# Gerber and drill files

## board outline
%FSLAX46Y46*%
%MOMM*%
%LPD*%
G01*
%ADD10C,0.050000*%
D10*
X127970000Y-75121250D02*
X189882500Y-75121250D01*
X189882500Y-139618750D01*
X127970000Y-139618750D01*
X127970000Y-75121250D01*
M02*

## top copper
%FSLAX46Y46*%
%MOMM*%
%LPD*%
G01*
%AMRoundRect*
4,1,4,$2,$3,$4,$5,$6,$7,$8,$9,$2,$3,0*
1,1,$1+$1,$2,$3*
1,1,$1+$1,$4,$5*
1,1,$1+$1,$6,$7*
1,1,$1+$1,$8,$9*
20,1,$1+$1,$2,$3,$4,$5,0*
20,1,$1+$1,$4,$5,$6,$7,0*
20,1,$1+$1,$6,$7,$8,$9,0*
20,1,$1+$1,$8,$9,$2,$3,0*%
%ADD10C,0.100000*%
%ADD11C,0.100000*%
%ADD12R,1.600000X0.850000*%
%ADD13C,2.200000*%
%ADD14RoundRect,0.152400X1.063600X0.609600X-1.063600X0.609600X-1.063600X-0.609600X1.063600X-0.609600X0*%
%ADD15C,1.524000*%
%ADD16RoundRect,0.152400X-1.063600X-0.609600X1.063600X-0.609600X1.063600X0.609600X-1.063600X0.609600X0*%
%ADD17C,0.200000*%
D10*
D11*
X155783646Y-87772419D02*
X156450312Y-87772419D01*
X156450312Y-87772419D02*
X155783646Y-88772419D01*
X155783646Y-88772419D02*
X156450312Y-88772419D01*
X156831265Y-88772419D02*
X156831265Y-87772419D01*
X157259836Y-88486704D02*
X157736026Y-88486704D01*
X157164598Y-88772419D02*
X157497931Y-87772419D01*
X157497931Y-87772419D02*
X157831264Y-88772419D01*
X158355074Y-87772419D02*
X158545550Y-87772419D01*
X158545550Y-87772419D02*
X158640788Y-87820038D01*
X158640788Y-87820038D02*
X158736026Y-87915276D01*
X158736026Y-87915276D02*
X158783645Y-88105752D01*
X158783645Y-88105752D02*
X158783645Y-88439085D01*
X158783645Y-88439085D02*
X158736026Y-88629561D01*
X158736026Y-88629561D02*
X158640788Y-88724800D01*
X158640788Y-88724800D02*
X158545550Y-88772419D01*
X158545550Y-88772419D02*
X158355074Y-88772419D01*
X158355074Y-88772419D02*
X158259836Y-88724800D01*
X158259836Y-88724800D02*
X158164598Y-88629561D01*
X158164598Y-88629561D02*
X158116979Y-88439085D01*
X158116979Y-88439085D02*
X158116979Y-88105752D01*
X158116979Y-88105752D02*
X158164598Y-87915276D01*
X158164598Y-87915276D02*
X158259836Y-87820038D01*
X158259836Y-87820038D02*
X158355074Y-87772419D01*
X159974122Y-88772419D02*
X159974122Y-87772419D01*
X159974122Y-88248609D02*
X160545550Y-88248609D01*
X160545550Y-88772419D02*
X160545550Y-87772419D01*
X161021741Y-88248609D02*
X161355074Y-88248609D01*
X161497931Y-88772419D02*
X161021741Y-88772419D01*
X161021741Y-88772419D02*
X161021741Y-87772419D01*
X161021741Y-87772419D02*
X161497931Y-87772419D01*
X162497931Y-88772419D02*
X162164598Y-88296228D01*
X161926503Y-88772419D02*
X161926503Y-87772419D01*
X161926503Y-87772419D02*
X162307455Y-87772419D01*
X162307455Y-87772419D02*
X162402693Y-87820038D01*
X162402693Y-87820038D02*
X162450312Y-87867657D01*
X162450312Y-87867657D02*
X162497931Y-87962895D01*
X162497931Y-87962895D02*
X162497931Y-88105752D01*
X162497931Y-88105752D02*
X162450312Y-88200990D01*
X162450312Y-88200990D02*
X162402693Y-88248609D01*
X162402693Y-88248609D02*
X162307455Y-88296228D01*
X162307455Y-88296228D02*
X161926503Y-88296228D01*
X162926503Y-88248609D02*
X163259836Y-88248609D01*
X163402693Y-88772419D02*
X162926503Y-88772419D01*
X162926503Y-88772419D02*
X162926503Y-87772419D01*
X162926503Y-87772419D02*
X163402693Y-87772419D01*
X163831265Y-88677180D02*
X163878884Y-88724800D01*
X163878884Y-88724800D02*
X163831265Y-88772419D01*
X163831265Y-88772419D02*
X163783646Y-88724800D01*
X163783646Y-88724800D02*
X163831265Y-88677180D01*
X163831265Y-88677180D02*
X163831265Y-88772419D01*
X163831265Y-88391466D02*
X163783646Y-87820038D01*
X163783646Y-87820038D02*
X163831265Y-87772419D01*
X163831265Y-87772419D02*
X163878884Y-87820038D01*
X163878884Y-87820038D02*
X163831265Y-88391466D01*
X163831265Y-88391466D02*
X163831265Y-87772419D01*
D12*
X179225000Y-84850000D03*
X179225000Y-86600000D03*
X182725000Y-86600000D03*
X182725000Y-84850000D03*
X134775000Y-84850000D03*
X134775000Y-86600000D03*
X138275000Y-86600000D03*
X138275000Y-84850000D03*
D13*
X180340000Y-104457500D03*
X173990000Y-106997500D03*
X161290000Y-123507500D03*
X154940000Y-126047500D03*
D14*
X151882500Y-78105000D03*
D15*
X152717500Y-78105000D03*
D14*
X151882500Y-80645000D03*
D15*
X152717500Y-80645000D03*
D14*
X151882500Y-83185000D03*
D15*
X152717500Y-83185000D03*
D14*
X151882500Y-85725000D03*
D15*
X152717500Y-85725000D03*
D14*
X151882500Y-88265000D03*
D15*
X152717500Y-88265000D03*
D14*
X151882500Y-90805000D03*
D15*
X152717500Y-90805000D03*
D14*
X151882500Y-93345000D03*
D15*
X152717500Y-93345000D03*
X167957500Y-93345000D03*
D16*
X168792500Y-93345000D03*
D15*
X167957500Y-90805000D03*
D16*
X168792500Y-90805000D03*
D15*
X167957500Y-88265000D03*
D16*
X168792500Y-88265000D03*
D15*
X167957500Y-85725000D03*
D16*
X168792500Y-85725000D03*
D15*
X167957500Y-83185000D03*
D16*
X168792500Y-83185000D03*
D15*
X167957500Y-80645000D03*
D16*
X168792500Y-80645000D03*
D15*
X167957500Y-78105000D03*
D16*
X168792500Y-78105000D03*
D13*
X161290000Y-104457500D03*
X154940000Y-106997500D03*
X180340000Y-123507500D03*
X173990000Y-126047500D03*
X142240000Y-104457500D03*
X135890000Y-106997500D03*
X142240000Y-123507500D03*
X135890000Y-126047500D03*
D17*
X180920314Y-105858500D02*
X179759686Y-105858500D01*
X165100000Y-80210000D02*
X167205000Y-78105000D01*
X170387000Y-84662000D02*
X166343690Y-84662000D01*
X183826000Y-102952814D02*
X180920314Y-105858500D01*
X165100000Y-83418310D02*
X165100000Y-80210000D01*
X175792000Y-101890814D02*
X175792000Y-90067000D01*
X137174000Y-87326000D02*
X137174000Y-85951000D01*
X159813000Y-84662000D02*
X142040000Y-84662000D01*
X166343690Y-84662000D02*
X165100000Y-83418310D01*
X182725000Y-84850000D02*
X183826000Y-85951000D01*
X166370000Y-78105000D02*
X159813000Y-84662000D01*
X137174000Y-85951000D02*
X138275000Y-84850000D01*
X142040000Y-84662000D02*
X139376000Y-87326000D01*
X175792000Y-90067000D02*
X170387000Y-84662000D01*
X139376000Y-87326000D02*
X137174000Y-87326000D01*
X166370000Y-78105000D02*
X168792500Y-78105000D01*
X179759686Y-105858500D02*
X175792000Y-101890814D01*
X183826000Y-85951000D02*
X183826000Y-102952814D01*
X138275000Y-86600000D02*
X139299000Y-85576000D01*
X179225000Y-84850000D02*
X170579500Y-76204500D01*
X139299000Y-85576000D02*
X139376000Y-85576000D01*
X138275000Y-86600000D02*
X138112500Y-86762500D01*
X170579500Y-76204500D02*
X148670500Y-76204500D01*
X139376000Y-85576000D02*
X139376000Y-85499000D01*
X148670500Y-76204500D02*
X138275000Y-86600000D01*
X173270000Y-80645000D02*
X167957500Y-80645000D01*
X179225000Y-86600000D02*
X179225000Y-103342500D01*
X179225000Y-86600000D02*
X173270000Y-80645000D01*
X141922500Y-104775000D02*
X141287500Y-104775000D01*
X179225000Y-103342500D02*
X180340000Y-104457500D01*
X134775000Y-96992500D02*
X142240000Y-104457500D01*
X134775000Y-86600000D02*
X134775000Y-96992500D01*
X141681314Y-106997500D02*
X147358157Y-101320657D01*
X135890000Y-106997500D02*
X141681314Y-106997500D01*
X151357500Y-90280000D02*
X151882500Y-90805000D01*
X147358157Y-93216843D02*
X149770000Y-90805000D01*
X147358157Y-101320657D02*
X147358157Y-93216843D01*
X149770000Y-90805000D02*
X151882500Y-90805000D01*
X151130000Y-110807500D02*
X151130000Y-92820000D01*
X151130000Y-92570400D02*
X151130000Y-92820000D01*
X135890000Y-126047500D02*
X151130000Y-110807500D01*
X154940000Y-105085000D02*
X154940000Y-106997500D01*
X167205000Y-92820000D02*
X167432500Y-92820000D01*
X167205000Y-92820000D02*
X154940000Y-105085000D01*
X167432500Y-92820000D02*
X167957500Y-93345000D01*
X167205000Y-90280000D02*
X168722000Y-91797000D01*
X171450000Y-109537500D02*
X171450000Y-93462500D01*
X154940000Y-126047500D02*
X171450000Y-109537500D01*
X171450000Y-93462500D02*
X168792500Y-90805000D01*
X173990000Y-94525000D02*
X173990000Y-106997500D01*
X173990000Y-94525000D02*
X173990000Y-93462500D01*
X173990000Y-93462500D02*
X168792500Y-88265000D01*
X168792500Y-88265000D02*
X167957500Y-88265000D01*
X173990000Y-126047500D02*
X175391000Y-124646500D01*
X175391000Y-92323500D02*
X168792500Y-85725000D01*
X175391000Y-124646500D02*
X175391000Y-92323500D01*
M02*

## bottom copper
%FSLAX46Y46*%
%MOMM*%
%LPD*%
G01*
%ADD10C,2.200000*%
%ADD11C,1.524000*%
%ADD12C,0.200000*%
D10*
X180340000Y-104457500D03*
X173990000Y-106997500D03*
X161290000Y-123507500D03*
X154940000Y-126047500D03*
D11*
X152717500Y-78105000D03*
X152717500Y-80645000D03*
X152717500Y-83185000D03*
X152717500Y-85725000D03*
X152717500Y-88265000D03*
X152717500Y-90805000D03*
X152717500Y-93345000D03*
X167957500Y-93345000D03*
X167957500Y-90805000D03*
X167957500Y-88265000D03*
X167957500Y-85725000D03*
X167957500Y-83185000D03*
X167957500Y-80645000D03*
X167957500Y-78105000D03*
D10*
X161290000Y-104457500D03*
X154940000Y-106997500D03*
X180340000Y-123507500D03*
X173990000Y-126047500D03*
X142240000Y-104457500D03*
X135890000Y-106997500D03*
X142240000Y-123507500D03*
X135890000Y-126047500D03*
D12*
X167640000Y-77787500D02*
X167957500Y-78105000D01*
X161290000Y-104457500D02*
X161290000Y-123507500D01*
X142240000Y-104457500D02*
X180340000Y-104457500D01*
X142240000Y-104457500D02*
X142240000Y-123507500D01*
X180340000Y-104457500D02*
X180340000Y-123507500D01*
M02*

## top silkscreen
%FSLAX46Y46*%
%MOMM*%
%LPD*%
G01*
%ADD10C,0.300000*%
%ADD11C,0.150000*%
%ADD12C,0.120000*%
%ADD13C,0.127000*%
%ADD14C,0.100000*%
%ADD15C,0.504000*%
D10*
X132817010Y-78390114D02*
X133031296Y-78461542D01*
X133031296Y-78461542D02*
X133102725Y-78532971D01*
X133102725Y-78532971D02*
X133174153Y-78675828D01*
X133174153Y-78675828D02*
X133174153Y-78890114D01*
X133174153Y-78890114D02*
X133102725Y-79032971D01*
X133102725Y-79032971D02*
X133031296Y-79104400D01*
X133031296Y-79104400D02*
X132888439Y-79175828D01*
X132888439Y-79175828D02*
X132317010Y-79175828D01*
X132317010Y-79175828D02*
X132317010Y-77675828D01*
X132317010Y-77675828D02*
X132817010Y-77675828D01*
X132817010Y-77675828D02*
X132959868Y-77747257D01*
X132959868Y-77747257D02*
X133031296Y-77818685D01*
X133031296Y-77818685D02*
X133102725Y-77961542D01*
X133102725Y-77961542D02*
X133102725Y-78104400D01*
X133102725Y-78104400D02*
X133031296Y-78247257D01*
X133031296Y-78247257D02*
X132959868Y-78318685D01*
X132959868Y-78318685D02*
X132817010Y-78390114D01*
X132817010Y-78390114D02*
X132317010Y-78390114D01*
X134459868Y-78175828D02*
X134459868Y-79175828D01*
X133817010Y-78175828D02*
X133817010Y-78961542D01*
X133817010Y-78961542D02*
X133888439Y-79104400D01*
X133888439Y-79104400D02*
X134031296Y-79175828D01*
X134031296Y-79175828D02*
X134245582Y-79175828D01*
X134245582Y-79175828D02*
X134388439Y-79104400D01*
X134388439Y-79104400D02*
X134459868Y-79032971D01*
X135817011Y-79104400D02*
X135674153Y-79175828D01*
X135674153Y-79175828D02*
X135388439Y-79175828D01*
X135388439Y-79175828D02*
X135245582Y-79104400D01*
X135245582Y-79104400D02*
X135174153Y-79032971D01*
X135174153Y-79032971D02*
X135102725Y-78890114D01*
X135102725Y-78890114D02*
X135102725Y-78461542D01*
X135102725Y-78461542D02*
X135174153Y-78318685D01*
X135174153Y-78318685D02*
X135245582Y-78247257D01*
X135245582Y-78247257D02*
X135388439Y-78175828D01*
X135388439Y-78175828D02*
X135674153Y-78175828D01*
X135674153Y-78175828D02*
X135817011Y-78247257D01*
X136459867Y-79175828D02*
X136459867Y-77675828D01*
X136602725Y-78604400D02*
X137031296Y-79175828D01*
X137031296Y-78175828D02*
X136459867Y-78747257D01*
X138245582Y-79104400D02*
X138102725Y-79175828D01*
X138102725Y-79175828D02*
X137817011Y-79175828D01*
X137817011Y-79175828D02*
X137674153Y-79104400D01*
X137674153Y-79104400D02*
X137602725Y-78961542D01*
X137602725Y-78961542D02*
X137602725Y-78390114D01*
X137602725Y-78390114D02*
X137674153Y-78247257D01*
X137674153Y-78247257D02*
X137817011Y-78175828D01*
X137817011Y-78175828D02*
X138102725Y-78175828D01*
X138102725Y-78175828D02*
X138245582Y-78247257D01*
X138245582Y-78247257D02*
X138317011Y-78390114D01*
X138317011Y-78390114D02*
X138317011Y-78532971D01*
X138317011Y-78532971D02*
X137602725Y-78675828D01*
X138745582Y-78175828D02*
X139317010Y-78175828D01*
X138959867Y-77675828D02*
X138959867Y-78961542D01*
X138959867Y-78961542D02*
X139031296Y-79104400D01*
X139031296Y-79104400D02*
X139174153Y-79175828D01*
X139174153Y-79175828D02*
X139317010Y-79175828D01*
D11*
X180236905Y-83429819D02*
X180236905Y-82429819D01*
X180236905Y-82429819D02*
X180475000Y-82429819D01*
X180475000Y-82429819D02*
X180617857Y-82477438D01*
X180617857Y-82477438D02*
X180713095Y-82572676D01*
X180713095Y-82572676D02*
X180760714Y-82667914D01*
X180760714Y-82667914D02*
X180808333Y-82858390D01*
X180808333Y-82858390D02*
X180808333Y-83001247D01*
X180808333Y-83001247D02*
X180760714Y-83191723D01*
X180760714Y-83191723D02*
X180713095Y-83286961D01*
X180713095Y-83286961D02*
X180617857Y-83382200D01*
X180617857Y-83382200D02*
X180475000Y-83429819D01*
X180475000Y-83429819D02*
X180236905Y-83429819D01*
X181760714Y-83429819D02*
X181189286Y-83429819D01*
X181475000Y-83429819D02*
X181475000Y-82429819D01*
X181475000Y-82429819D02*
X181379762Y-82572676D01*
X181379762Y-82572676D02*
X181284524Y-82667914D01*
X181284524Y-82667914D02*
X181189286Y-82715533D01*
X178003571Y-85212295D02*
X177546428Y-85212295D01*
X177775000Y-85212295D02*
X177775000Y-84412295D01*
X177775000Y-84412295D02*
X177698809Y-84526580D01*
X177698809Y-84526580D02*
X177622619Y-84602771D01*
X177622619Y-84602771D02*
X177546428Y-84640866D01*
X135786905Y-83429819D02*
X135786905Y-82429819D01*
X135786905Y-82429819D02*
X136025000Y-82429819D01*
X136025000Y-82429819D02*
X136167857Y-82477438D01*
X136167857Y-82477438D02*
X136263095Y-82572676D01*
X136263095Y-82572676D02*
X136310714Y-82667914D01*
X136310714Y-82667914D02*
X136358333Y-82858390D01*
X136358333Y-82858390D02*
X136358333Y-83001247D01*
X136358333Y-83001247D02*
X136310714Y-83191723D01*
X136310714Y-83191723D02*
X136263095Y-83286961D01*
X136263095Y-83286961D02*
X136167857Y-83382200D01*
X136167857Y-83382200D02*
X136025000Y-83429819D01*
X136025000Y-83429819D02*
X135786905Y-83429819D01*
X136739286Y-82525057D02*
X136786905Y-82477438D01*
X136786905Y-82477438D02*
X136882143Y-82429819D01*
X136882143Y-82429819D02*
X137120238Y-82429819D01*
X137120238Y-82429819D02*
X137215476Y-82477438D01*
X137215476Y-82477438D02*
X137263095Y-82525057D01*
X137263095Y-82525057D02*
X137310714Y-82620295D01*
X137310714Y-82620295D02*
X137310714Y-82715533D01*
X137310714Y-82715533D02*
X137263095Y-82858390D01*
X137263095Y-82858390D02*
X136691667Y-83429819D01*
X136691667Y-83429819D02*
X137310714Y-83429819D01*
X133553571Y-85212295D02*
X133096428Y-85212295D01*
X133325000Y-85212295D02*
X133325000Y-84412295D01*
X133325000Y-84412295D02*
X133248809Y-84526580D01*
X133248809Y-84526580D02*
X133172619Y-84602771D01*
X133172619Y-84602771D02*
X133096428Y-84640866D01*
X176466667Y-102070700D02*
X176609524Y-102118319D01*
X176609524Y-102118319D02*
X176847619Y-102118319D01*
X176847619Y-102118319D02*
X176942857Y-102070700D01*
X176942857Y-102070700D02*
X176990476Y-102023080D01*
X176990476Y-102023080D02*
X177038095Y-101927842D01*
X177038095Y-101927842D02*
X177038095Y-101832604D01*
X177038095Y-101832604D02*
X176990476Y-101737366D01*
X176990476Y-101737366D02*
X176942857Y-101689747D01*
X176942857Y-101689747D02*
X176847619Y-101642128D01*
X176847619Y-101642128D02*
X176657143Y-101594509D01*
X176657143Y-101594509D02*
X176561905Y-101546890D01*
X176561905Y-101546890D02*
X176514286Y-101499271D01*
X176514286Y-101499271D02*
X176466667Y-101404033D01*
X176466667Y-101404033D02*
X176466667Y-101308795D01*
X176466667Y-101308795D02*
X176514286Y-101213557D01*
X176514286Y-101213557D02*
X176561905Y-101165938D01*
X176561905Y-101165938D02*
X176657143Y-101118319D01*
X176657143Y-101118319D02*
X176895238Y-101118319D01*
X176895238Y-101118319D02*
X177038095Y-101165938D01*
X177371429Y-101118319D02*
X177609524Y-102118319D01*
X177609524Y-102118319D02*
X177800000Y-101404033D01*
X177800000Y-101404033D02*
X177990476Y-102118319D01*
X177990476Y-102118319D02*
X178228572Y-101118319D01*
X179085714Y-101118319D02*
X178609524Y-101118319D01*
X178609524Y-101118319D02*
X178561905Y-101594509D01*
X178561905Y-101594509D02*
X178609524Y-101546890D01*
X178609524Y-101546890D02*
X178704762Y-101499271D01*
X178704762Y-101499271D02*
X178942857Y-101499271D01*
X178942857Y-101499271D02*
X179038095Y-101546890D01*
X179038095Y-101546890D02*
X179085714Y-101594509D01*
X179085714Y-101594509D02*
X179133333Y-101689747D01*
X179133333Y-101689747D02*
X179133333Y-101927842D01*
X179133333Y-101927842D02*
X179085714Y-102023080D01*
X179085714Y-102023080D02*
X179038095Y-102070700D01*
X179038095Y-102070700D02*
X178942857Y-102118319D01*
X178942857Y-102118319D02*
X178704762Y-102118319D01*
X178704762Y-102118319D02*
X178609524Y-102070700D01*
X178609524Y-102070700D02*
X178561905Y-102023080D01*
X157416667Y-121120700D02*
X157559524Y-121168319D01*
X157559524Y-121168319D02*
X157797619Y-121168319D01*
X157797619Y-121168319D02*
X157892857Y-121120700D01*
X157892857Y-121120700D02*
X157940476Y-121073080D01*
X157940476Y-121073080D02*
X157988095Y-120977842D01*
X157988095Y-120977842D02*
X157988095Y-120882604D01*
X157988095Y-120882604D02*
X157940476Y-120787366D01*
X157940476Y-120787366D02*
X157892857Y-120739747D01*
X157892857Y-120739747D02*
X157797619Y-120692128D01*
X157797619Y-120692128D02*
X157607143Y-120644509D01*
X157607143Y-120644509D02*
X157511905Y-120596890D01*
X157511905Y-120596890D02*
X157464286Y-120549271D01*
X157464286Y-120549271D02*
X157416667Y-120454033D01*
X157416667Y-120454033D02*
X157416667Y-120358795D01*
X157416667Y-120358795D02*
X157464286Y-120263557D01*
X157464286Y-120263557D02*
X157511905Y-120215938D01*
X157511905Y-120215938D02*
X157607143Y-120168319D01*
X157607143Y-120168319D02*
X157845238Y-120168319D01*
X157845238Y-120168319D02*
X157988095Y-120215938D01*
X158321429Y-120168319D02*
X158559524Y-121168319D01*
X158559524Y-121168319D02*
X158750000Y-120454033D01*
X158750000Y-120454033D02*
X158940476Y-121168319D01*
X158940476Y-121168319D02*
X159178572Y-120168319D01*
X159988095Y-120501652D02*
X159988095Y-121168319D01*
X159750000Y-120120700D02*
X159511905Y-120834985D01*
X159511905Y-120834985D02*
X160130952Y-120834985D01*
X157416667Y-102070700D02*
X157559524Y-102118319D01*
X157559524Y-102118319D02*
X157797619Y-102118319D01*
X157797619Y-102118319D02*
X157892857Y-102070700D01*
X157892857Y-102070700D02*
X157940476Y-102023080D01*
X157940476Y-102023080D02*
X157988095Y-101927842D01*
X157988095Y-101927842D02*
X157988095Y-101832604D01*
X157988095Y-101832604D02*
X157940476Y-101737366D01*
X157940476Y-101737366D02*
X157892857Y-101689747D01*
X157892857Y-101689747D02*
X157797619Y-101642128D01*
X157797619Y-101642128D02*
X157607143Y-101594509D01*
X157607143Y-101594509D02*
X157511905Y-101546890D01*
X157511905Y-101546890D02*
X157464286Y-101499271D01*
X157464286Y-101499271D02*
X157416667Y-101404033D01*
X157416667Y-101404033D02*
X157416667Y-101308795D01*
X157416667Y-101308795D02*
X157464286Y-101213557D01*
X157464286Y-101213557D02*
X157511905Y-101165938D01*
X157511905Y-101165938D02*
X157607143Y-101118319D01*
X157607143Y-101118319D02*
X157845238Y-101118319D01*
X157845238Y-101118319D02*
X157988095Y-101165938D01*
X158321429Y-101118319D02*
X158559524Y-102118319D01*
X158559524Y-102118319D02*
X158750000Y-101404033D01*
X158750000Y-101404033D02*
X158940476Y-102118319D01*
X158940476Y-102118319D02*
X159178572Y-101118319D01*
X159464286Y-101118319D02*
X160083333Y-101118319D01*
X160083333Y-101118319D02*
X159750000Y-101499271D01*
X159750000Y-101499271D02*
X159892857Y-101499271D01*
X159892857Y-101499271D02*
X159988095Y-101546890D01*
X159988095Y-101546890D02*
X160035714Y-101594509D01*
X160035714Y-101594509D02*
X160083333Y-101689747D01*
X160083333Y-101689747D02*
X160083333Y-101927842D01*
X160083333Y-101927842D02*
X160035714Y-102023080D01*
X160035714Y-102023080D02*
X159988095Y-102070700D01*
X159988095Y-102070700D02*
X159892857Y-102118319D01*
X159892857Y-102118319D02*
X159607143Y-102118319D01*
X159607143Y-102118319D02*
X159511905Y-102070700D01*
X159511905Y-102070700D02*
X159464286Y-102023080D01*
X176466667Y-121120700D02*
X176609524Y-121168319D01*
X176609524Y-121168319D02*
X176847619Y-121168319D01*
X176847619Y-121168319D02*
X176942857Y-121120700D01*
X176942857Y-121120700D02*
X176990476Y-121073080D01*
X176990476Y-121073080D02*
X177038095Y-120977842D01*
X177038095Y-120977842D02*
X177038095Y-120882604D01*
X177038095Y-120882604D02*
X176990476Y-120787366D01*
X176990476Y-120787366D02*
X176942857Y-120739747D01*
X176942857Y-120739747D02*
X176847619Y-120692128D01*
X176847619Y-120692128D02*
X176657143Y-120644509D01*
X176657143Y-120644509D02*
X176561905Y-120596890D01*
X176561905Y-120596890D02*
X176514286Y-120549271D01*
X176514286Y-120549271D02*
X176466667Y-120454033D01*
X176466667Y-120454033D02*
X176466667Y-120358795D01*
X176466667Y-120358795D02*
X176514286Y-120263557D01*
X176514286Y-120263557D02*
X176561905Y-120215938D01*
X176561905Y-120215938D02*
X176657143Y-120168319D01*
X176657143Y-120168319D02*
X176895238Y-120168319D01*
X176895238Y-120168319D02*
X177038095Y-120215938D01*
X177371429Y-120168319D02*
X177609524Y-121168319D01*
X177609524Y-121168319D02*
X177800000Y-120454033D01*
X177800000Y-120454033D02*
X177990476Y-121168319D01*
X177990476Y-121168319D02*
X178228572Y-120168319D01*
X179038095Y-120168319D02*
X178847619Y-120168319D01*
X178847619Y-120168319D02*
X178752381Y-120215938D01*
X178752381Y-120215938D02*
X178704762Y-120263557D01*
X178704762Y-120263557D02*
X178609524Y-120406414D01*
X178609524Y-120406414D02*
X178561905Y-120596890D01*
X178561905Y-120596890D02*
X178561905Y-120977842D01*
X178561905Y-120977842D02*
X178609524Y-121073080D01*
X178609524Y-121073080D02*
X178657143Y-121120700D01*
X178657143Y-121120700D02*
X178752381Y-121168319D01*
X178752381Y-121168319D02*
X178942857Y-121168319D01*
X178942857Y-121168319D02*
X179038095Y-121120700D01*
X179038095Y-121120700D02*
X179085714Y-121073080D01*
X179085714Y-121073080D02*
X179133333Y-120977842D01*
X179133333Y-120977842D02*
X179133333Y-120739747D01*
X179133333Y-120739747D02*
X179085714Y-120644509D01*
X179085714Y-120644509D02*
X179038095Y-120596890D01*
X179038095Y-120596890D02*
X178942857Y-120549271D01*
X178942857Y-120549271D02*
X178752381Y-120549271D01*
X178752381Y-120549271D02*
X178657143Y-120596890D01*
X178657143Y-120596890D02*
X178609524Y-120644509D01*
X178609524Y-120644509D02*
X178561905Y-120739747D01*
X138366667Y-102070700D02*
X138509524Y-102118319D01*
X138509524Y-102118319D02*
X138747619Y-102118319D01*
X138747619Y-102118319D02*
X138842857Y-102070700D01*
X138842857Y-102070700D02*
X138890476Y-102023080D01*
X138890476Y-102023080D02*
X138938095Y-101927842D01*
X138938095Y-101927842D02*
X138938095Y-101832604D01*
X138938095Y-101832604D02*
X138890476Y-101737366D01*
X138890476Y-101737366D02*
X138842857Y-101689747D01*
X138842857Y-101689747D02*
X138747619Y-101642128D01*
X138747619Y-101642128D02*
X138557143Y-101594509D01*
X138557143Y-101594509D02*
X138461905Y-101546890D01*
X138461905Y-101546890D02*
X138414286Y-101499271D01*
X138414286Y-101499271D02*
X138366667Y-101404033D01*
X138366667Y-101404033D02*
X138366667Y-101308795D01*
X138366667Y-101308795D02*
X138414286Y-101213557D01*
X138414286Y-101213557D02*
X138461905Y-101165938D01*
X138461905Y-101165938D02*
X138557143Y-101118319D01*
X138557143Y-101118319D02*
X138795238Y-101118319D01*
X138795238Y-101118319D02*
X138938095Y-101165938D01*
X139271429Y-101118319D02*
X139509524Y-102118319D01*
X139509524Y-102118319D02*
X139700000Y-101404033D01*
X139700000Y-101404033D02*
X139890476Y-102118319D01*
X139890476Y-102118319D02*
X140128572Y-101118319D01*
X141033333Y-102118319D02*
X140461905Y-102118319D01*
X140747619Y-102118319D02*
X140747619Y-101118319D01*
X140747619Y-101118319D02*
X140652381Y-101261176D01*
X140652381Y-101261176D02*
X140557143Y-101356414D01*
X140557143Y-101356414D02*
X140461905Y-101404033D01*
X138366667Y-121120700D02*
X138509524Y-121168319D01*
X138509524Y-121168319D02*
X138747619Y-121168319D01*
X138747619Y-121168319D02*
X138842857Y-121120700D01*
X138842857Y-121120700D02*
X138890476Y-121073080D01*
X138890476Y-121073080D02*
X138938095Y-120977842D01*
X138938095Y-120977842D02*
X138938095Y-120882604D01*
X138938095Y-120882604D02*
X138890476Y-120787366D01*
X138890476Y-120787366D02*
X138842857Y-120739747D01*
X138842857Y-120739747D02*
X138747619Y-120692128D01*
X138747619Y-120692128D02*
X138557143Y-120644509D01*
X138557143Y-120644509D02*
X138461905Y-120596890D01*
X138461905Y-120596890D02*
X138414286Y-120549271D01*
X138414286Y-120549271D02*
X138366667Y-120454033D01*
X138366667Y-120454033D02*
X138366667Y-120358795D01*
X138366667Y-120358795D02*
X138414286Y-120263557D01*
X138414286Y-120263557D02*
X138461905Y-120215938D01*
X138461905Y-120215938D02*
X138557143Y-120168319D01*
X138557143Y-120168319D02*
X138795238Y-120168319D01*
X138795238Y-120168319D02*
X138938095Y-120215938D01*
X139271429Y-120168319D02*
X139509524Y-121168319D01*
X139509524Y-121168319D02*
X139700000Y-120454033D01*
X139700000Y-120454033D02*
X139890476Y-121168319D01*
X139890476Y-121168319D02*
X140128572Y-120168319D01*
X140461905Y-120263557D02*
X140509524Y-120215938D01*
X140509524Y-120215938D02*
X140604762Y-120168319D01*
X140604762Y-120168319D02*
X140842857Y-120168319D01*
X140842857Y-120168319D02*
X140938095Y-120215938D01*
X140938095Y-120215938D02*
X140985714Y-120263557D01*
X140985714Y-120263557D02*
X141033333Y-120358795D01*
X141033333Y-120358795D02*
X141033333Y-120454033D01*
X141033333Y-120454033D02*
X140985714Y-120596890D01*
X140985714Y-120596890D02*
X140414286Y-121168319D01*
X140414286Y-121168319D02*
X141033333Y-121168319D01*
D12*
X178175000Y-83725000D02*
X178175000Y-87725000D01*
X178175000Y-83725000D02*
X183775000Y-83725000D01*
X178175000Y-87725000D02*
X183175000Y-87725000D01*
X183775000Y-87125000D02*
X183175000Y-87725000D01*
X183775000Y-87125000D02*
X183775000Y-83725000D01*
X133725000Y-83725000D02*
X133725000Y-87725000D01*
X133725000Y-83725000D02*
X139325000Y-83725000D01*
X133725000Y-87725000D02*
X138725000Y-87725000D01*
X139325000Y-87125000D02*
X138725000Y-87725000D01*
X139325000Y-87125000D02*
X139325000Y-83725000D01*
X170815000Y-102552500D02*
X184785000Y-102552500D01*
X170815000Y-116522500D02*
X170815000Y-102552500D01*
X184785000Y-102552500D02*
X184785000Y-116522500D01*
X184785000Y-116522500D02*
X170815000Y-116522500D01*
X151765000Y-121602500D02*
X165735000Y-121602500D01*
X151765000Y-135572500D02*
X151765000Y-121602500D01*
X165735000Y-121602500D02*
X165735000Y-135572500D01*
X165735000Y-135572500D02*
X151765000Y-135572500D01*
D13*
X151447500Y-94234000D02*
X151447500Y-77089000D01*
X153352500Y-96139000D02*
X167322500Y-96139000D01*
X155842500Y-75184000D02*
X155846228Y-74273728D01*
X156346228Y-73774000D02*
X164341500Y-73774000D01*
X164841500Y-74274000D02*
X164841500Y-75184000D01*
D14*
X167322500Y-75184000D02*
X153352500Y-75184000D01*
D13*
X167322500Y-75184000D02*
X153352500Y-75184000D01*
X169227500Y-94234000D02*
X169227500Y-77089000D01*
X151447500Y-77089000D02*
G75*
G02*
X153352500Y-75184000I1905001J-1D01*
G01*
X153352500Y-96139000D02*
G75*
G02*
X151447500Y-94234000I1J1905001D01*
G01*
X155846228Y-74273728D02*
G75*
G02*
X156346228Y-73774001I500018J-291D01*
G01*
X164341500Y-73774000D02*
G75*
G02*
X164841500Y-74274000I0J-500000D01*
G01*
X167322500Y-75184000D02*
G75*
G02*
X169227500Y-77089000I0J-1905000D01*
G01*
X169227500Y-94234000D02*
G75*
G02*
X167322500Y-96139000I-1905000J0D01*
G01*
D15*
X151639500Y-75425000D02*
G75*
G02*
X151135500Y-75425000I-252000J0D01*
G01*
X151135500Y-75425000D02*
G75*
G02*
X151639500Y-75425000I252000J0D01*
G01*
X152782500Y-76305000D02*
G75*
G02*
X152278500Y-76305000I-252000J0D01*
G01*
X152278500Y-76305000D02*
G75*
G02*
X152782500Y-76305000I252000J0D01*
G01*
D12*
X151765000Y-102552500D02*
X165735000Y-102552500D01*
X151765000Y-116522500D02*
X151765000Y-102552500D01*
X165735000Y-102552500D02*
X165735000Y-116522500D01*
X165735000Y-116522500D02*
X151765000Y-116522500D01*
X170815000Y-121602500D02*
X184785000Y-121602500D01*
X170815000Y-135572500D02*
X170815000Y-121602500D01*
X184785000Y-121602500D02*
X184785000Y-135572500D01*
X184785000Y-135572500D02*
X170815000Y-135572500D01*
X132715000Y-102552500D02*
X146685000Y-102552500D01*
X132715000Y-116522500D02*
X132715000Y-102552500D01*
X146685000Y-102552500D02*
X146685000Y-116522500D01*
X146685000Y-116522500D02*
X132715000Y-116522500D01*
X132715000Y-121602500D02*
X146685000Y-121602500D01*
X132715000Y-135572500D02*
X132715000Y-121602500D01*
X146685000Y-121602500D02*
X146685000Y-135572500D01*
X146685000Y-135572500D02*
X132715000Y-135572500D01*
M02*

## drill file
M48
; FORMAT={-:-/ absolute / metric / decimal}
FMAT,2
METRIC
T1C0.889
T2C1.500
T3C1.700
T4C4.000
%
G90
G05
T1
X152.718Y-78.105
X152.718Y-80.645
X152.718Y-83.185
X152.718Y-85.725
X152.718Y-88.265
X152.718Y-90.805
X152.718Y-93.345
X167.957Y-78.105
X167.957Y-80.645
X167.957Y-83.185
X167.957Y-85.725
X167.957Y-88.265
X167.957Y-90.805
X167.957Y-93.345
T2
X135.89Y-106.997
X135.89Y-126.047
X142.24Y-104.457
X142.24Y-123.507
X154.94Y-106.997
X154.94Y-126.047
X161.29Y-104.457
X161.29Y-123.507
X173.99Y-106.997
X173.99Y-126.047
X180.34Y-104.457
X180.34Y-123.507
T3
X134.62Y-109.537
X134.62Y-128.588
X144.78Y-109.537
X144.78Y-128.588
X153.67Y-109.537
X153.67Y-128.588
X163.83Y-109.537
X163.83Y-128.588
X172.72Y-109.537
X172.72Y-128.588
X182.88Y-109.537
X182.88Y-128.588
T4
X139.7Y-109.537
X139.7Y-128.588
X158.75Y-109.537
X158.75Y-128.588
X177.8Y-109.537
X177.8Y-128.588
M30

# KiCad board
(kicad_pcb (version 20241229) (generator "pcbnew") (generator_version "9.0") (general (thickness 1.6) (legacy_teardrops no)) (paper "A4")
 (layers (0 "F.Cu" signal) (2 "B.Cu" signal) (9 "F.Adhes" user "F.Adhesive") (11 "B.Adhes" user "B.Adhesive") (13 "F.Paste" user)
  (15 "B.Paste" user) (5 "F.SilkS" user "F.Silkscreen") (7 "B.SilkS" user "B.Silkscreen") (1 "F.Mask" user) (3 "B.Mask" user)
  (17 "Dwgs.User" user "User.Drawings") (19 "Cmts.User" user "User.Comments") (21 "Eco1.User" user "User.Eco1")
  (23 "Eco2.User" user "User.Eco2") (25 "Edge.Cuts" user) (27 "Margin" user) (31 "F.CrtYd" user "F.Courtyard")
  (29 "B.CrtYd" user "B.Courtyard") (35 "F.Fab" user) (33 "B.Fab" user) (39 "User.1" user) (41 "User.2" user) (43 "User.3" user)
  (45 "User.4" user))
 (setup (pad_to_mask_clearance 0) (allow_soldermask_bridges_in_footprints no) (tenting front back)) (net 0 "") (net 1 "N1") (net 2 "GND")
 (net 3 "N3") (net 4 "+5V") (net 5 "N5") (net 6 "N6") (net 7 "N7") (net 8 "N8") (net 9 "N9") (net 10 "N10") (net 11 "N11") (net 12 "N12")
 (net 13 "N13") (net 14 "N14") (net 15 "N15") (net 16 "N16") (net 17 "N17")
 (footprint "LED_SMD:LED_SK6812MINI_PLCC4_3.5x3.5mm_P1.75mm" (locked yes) (layer "F.Cu") (at 180.975 85.725)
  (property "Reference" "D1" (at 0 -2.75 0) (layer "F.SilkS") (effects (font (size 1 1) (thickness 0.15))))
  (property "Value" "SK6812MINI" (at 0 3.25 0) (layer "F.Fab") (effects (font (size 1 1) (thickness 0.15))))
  (fp_line (start -2.8 -2) (end -2.8 2) (stroke (width 0.12) (type default)) (layer "F.SilkS"))
  (fp_line (start -2.8 -2) (end 2.8 -2) (stroke (width 0.12) (type solid)) (layer "F.SilkS"))
  (fp_line (start -2.8 2) (end 2.2 2) (stroke (width 0.12) (type solid)) (layer "F.SilkS"))
  (fp_line (start 2.8 1.4) (end 2.2 2) (stroke (width 0.12) (type default)) (layer "F.SilkS"))
  (fp_line (start 2.8 1.4) (end 2.8 -2) (stroke (width 0.12) (type solid)) (layer "F.SilkS"))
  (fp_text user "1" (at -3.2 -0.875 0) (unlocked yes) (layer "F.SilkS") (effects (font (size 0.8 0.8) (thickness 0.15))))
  (pad "1" smd rect (at -1.75 -0.875) (size 1.6 0.85) (layers "F.Cu" "F.Mask" "F.Paste") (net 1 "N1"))
  (pad "2" smd rect (at -1.75 0.875) (size 1.6 0.85) (layers "F.Cu" "F.Mask" "F.Paste") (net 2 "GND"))
  (pad "3" smd rect (at 1.75 0.875) (size 1.6 0.85) (layers "F.Cu" "F.Mask" "F.Paste") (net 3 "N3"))
  (pad "4" smd rect (at 1.75 -0.875) (size 1.6 0.85) (layers "F.Cu" "F.Mask" "F.Paste") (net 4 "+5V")))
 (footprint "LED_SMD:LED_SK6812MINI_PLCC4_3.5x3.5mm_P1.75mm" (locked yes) (layer "F.Cu") (at 136.525 85.725)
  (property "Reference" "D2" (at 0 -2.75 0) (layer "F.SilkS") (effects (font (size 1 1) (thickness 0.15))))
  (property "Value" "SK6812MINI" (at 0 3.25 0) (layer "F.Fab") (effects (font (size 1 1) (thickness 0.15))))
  (fp_line (start -2.8 -2) (end -2.8 2) (stroke (width 0.12) (type default)) (layer "F.SilkS"))
  (fp_line (start -2.8 -2) (end 2.8 -2) (stroke (width 0.12) (type solid)) (layer "F.SilkS"))
  (fp_line (start -2.8 2) (end 2.2 2) (stroke (width 0.12) (type solid)) (layer "F.SilkS"))
  (fp_line (start 2.8 1.4) (end 2.2 2) (stroke (width 0.12) (type default)) (layer "F.SilkS"))
  (fp_line (start 2.8 1.4) (end 2.8 -2) (stroke (width 0.12) (type solid)) (layer "F.SilkS"))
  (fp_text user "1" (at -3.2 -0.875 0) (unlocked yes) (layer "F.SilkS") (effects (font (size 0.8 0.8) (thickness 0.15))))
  (pad "1" smd rect (at -1.75 -0.875) (size 1.6 0.85) (layers "F.Cu" "F.Mask" "F.Paste") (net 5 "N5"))
  (pad "2" smd rect (at -1.75 0.875) (size 1.6 0.85) (layers "F.Cu" "F.Mask" "F.Paste") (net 2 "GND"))
  (pad "3" smd rect (at 1.75 0.875) (size 1.6 0.85) (layers "F.Cu" "F.Mask" "F.Paste") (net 1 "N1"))
  (pad "4" smd rect (at 1.75 -0.875) (size 1.6 0.85) (layers "F.Cu" "F.Mask" "F.Paste") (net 4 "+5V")))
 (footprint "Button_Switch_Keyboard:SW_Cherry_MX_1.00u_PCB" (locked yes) (layer "F.Cu") (at 180.34 104.4575)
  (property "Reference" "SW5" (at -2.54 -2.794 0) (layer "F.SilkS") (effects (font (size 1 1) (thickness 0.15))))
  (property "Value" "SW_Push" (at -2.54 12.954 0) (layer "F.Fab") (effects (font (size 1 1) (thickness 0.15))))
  (fp_line (start -9.525 -1.905) (end 4.445 -1.905) (stroke (width 0.12) (type solid)) (layer "F.SilkS"))
  (fp_line (start -9.525 12.065) (end -9.525 -1.905) (stroke (width 0.12) (type solid)) (layer "F.SilkS"))
  (fp_line (start 4.445 -1.905) (end 4.445 12.065) (stroke (width 0.12) (type solid)) (layer "F.SilkS"))
  (fp_line (start 4.445 12.065) (end -9.525 12.065) (stroke (width 0.12) (type solid)) (layer "F.SilkS"))
  (pad "" np_thru_hole circle (at -7.62 5.08) (size 1.7 1.7) (drill 1.7) (layers "*.Cu" "*.Mask"))
  (pad "" np_thru_hole circle (at -2.54 5.08) (size 4 4) (drill 4) (layers "*.Cu" "*.Mask"))
  (pad "" np_thru_hole circle (at 2.54 5.08) (size 1.7 1.7) (drill 1.7) (layers "*.Cu" "*.Mask"))
  (pad "1" thru_hole circle (at 0 0) (size 2.2 2.2) (drill 1.5) (layers "*.Cu" "*.Mask") (remove_unused_layers no) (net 2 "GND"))
  (pad "2" thru_hole circle (at -6.35 2.54) (size 2.2 2.2) (drill 1.5) (layers "*.Cu" "*.Mask") (remove_unused_layers no) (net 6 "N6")))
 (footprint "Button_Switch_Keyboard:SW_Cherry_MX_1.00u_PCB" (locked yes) (layer "F.Cu") (at 161.29 123.5075)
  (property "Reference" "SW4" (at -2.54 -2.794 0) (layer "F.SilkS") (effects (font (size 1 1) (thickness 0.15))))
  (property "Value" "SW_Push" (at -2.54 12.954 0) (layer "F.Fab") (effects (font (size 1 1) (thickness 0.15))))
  (fp_line (start -9.525 -1.905) (end 4.445 -1.905) (stroke (width 0.12) (type solid)) (layer "F.SilkS"))
  (fp_line (start -9.525 12.065) (end -9.525 -1.905) (stroke (width 0.12) (type solid)) (layer "F.SilkS"))
  (fp_line (start 4.445 -1.905) (end 4.445 12.065) (stroke (width 0.12) (type solid)) (layer "F.SilkS"))
  (fp_line (start 4.445 12.065) (end -9.525 12.065) (stroke (width 0.12) (type solid)) (layer "F.SilkS"))
  (pad "" np_thru_hole circle (at -7.62 5.08) (size 1.7 1.7) (drill 1.7) (layers "*.Cu" "*.Mask"))
  (pad "" np_thru_hole circle (at -2.54 5.08) (size 4 4) (drill 4) (layers "*.Cu" "*.Mask"))
  (pad "" np_thru_hole circle (at 2.54 5.08) (size 1.7 1.7) (drill 1.7) (layers "*.Cu" "*.Mask"))
  (pad "1" thru_hole circle (at 0 0) (size 2.2 2.2) (drill 1.5) (layers "*.Cu" "*.Mask") (remove_unused_layers no) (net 2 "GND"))
  (pad "2" thru_hole circle (at -6.35 2.54) (size 2.2 2.2) (drill 1.5) (layers "*.Cu" "*.Mask") (remove_unused_layers no) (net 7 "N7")))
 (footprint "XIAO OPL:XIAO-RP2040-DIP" (layer "F.Cu") (at 160.3375 85.725)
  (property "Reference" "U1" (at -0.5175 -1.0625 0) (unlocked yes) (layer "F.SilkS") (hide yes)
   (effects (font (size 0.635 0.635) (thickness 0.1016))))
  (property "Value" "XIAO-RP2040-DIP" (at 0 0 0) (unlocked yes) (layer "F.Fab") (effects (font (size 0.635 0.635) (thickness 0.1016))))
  (fp_line (start -8.89 8.509) (end -8.89 -8.636) (stroke (width 0.127) (type solid)) (layer "F.SilkS"))
  (fp_line (start -6.985 10.414) (end 6.985 10.414) (stroke (width 0.127) (type solid)) (layer "F.SilkS"))
  (fp_line (start -4.495 -10.541) (end -4.491272 -11.451272) (stroke (width 0.127) (type solid)) (layer "F.SilkS"))
  (fp_line (start -3.991272 -11.951) (end 4.004 -11.951) (stroke (width 0.127) (type solid)) (layer "F.SilkS"))
  (fp_line (start 4.504 -11.451) (end 4.504 -10.541) (stroke (width 0.127) (type solid)) (layer "F.SilkS"))
  (fp_line (start 6.985 -10.541) (end -6.985 -10.541) (stroke (width 0.1) (type solid)) (layer "F.SilkS"))
  (fp_line (start 6.985 -10.541) (end -6.985 -10.541) (stroke (width 0.127) (type solid)) (layer "F.SilkS"))
  (fp_line (start 8.89 8.509) (end 8.89 -8.636) (stroke (width 0.127) (type solid)) (layer "F.SilkS"))
  (fp_arc (start -8.89 -8.636) (mid -8.332038 -9.983038) (end -6.985 -10.541) (stroke (width 0.127) (type solid)) (layer "F.SilkS"))
  (fp_arc (start -6.985 10.414) (mid -8.332038 9.856038) (end -8.89 8.509) (stroke (width 0.127) (type solid)) (layer "F.SilkS"))
  (fp_arc (start -4.491272 -11.451272) (mid -4.344728 -11.80464) (end -3.991272 -11.951) (stroke (width 0.127) (type default))
   (layer "F.SilkS"))
  (fp_arc (start 4.004 -11.951) (mid 4.357553 -11.804553) (end 4.504 -11.451) (stroke (width 0.127) (type default)) (layer "F.SilkS"))
  (fp_arc (start 6.985 -10.541) (mid 8.332038 -9.983038) (end 8.89 -8.636) (stroke (width 0.127) (type solid)) (layer "F.SilkS"))
  (fp_arc (start 8.89 8.509) (mid 8.332038 9.856038) (end 6.985 10.414) (stroke (width 0.127) (type solid)) (layer "F.SilkS"))
  (fp_circle (center -8.95 -10.3) (end -8.95 -10.554) (stroke (width 0.5) (type solid)) (fill yes) (layer "F.SilkS"))
  (fp_circle (center -7.807 -9.42) (end -7.807 -9.674) (stroke (width 0.5) (type solid)) (fill yes) (layer "F.SilkS"))
  (pad "1" smd roundrect (at -8.455 -7.62 180) (size 2.432 1.524) (layers "F.Cu" "F.Mask") (roundrect_rratio 0.1) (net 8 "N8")
   (thermal_bridge_angle 45))
  (pad "1" thru_hole circle (at -7.62 -7.62 180) (size 1.524 1.524) (drill 0.889) (layers "*.Cu" "*.Mask") (remove_unused_layers no)
   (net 8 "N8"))
  (pad "2" smd roundrect (at -8.455 -5.08 180) (size 2.432 1.524) (layers "F.Cu" "F.Mask") (roundrect_rratio 0.1) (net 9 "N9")
   (thermal_bridge_angle 45))
  (pad "2" thru_hole circle (at -7.62 -5.08 180) (size 1.524 1.524) (drill 0.889) (layers "*.Cu" "*.Mask") (remove_unused_layers no)
   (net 9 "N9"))
  (pad "3" smd roundrect (at -8.455 -2.54 180) (size 2.432 1.524) (layers "F.Cu" "F.Mask") (roundrect_rratio 0.1) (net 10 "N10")
   (thermal_bridge_angle 45))
  (pad "3" thru_hole circle (at -7.62 -2.54 180) (size 1.524 1.524) (drill 0.889) (layers "*.Cu" "*.Mask") (remove_unused_layers no)
   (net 10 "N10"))
  (pad "4" smd roundrect (at -8.455 0 180) (size 2.432 1.524) (layers "F.Cu" "F.Mask") (roundrect_rratio 0.1) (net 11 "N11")
   (thermal_bridge_angle 45))
  (pad "4" thru_hole circle (at -7.62 0 180) (size 1.524 1.524) (drill 0.889) (layers "*.Cu" "*.Mask") (remove_unused_layers no)
   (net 11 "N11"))
  (pad "5" smd roundrect (at -8.455 2.54 180) (size 2.432 1.524) (layers "F.Cu" "F.Mask") (roundrect_rratio 0.1) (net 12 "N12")
   (thermal_bridge_angle 45))
  (pad "5" thru_hole circle (at -7.62 2.54 180) (size 1.524 1.524) (drill 0.889) (layers "*.Cu" "*.Mask") (remove_unused_layers no)
   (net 12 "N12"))
  (pad "6" smd roundrect (at -8.455 5.08 180) (size 2.432 1.524) (layers "F.Cu" "F.Mask") (roundrect_rratio 0.1) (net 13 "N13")
   (thermal_bridge_angle 45))
  (pad "6" thru_hole circle (at -7.62 5.08 180) (size 1.524 1.524) (drill 0.889) (layers "*.Cu" "*.Mask") (remove_unused_layers no)
   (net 13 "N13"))
  (pad "7" smd roundrect (at -8.455 7.62 180) (size 2.432 1.524) (layers "F.Cu" "F.Mask") (roundrect_rratio 0.1) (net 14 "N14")
   (thermal_bridge_angle 45))
  (pad "7" thru_hole circle (at -7.62 7.62 180) (size 1.524 1.524) (drill 0.889) (layers "*.Cu" "*.Mask") (remove_unused_layers no)
   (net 14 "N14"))
  (pad "8" thru_hole circle (at 7.62 7.62) (size 1.524 1.524) (drill 0.889) (layers "*.Cu" "*.Mask") (remove_unused_layers no)
   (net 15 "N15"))
  (pad "8" smd roundrect (at 8.455 7.62) (size 2.432 1.524) (layers "F.Cu" "F.Mask") (roundrect_rratio 0.1) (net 15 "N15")
   (thermal_bridge_angle 45))
  (pad "9" thru_hole circle (at 7.62 5.08) (size 1.524 1.524) (drill 0.889) (layers "*.Cu" "*.Mask") (remove_unused_layers no) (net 7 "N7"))
  (pad "9" smd roundrect (at 8.455 5.08) (size 2.432 1.524) (layers "F.Cu" "F.Mask") (roundrect_rratio 0.1) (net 7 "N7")
   (thermal_bridge_angle 45))
  (pad "10" thru_hole circle (at 7.62 2.54) (size 1.524 1.524) (drill 0.889) (layers "*.Cu" "*.Mask") (remove_unused_layers no) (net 6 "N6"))
  (pad "10" smd roundrect (at 8.455 2.54) (size 2.432 1.524) (layers "F.Cu" "F.Mask") (roundrect_rratio 0.1) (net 6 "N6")
   (thermal_bridge_angle 45))
  (pad "11" thru_hole circle (at 7.62 0) (size 1.524 1.524) (drill 0.889) (layers "*.Cu" "*.Mask") (remove_unused_layers no) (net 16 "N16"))
  (pad "11" smd roundrect (at 8.455 0) (size 2.432 1.524) (layers "F.Cu" "F.Mask") (roundrect_rratio 0.1) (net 16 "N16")
   (thermal_bridge_angle 45))
  (pad "12" thru_hole circle (at 7.62 -2.54) (size 1.524 1.524) (drill 0.889) (layers "*.Cu" "*.Mask") (remove_unused_layers no)
   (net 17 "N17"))
  (pad "12" smd roundrect (at 8.455 -2.54) (size 2.432 1.524) (layers "F.Cu" "F.Mask") (roundrect_rratio 0.1) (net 17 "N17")
   (thermal_bridge_angle 45))
  (pad "13" thru_hole circle (at 7.62 -5.08) (size 1.524 1.524) (drill 0.889) (layers "*.Cu" "*.Mask") (remove_unused_layers no)
   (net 2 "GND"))
  (pad "13" smd roundrect (at 8.455 -5.08) (size 2.432 1.524) (layers "F.Cu" "F.Mask") (roundrect_rratio 0.1) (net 2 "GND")
   (thermal_bridge_angle 45))
  (pad "14" thru_hole circle (at 7.62 -7.62) (size 1.524 1.524) (drill 0.889) (layers "*.Cu" "*.Mask") (remove_unused_layers no)
   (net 4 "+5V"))
  (pad "14" smd roundrect (at 8.455 -7.62) (size 2.432 1.524) (layers "F.Cu" "F.Mask") (roundrect_rratio 0.1) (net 4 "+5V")
   (thermal_bridge_angle 45)))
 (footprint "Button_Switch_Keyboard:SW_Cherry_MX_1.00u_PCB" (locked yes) (layer "F.Cu") (at 161.29 104.4575)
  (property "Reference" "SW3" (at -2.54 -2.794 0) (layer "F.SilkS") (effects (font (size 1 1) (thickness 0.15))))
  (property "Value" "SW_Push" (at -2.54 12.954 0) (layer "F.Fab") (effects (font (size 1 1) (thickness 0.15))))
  (fp_line (start -9.525 -1.905) (end 4.445 -1.905) (stroke (width 0.12) (type solid)) (layer "F.SilkS"))
  (fp_line (start -9.525 12.065) (end -9.525 -1.905) (stroke (width 0.12) (type solid)) (layer "F.SilkS"))
  (fp_line (start 4.445 -1.905) (end 4.445 12.065) (stroke (width 0.12) (type solid)) (layer "F.SilkS"))
  (fp_line (start 4.445 12.065) (end -9.525 12.065) (stroke (width 0.12) (type solid)) (layer "F.SilkS"))
  (pad "" np_thru_hole circle (at -7.62 5.08) (size 1.7 1.7) (drill 1.7) (layers "*.Cu" "*.Mask"))
  (pad "" np_thru_hole circle (at -2.54 5.08) (size 4 4) (drill 4) (layers "*.Cu" "*.Mask"))
  (pad "" np_thru_hole circle (at 2.54 5.08) (size 1.7 1.7) (drill 1.7) (layers "*.Cu" "*.Mask"))
  (pad "1" thru_hole circle (at 0 0) (size 2.2 2.2) (drill 1.5) (layers "*.Cu" "*.Mask") (remove_unused_layers no) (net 2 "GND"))
  (pad "2" thru_hole circle (at -6.35 2.54) (size 2.2 2.2) (drill 1.5) (layers "*.Cu" "*.Mask") (remove_unused_layers no) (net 15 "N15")))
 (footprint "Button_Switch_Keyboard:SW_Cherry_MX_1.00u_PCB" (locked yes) (layer "F.Cu") (at 180.34 123.5075)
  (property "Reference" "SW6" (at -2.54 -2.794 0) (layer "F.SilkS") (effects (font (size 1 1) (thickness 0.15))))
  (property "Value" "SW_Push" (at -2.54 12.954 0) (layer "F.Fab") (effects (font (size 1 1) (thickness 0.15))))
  (fp_line (start -9.525 -1.905) (end 4.445 -1.905) (stroke (width 0.12) (type solid)) (layer "F.SilkS"))
  (fp_line (start -9.525 12.065) (end -9.525 -1.905) (stroke (width 0.12) (type solid)) (layer "F.SilkS"))
  (fp_line (start 4.445 -1.905) (end 4.445 12.065) (stroke (width 0.12) (type solid)) (layer "F.SilkS"))
  (fp_line (start 4.445 12.065) (end -9.525 12.065) (stroke (width 0.12) (type solid)) (layer "F.SilkS"))
  (pad "" np_thru_hole circle (at -7.62 5.08) (size 1.7 1.7) (drill 1.7) (layers "*.Cu" "*.Mask"))
  (pad "" np_thru_hole circle (at -2.54 5.08) (size 4 4) (drill 4) (layers "*.Cu" "*.Mask"))
  (pad "" np_thru_hole circle (at 2.54 5.08) (size 1.7 1.7) (drill 1.7) (layers "*.Cu" "*.Mask"))
  (pad "1" thru_hole circle (at 0 0) (size 2.2 2.2) (drill 1.5) (layers "*.Cu" "*.Mask") (remove_unused_layers no) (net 2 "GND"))
  (pad "2" thru_hole circle (at -6.35 2.54) (size 2.2 2.2) (drill 1.5) (layers "*.Cu" "*.Mask") (remove_unused_layers no) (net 16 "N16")))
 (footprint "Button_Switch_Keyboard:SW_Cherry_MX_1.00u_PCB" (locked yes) (layer "F.Cu") (at 142.24 104.4575)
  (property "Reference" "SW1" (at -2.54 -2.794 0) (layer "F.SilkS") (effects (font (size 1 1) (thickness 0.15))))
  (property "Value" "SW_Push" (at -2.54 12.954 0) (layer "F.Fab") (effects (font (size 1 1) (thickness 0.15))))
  (fp_line (start -9.525 -1.905) (end 4.445 -1.905) (stroke (width 0.12) (type solid)) (layer "F.SilkS"))
  (fp_line (start -9.525 12.065) (end -9.525 -1.905) (stroke (width 0.12) (type solid)) (layer "F.SilkS"))
  (fp_line (start 4.445 -1.905) (end 4.445 12.065) (stroke (width 0.12) (type solid)) (layer "F.SilkS"))
  (fp_line (start 4.445 12.065) (end -9.525 12.065) (stroke (width 0.12) (type solid)) (layer "F.SilkS"))
  (pad "" np_thru_hole circle (at -7.62 5.08) (size 1.7 1.7) (drill 1.7) (layers "*.Cu" "*.Mask"))
  (pad "" np_thru_hole circle (at -2.54 5.08) (size 4 4) (drill 4) (layers "*.Cu" "*.Mask"))
  (pad "" np_thru_hole circle (at 2.54 5.08) (size 1.7 1.7) (drill 1.7) (layers "*.Cu" "*.Mask"))
  (pad "1" thru_hole circle (at 0 0) (size 2.2 2.2) (drill 1.5) (layers "*.Cu" "*.Mask") (remove_unused_layers no) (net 2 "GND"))
  (pad "2" thru_hole circle (at -6.35 2.54) (size 2.2 2.2) (drill 1.5) (layers "*.Cu" "*.Mask") (remove_unused_layers no) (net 13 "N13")))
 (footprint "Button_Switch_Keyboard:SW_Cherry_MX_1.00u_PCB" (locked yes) (layer "F.Cu") (at 142.24 123.5075)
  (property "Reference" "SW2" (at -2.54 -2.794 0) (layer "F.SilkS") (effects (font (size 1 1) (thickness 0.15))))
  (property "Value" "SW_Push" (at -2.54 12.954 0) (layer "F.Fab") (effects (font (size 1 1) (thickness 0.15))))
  (fp_line (start -9.525 -1.905) (end 4.445 -1.905) (stroke (width 0.12) (type solid)) (layer "F.SilkS"))
  (fp_line (start -9.525 12.065) (end -9.525 -1.905) (stroke (width 0.12) (type solid)) (layer "F.SilkS"))
  (fp_line (start 4.445 -1.905) (end 4.445 12.065) (stroke (width 0.12) (type solid)) (layer "F.SilkS"))
  (fp_line (start 4.445 12.065) (end -9.525 12.065) (stroke (width 0.12) (type solid)) (layer "F.SilkS"))
  (pad "" np_thru_hole circle (at -7.62 5.08) (size 1.7 1.7) (drill 1.7) (layers "*.Cu" "*.Mask"))
  (pad "" np_thru_hole circle (at -2.54 5.08) (size 4 4) (drill 4) (layers "*.Cu" "*.Mask"))
  (pad "" np_thru_hole circle (at 2.54 5.08) (size 1.7 1.7) (drill 1.7) (layers "*.Cu" "*.Mask"))
  (pad "1" thru_hole circle (at 0 0) (size 2.2 2.2) (drill 1.5) (layers "*.Cu" "*.Mask") (remove_unused_layers no) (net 2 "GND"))
  (pad "2" thru_hole circle (at -6.35 2.54) (size 2.2 2.2) (drill 1.5) (layers "*.Cu" "*.Mask") (remove_unused_layers no) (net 14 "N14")))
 (gr_rect (start 127.97 75.12125) (end 189.8825 139.61875) (stroke (width 0.05) (type solid)) (fill no) (layer "Edge.Cuts"))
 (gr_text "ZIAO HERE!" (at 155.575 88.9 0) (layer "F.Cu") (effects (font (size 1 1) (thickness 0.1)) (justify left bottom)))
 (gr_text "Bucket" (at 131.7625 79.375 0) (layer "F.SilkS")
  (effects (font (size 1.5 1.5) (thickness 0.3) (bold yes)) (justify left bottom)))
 (segment (start 180.920314 105.8585) (end 179.759686 105.8585) (width 0.2) (layer "F.Cu") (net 4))
 (segment (start 165.1 80.21) (end 167.205 78.105) (width 0.2) (layer "F.Cu") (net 4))
 (segment (start 170.387 84.662) (end 166.34369 84.662) (width 0.2) (layer "F.Cu") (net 4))
 (segment (start 183.826 102.952814) (end 180.920314 105.8585) (width 0.2) (layer "F.Cu") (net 4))
 (segment (start 165.1 83.41831) (end 165.1 80.21) (width 0.2) (layer "F.Cu") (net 4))
 (segment (start 175.792 101.890814) (end 175.792 90.067) (width 0.2) (layer "F.Cu") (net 4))
 (segment (start 137.174 87.326) (end 137.174 85.951) (width 0.2) (layer "F.Cu") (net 4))
 (segment (start 159.813 84.662) (end 142.04 84.662) (width 0.2) (layer "F.Cu") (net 4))
 (segment (start 166.34369 84.662) (end 165.1 83.41831) (width 0.2) (layer "F.Cu") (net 4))
 (segment (start 182.725 84.85) (end 183.826 85.951) (width 0.2) (layer "F.Cu") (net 4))
 (segment (start 166.37 78.105) (end 159.813 84.662) (width 0.2) (layer "F.Cu") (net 4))
 (segment (start 137.174 85.951) (end 138.275 84.85) (width 0.2) (layer "F.Cu") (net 4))
 (segment (start 142.04 84.662) (end 139.376 87.326) (width 0.2) (layer "F.Cu") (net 4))
 (segment (start 175.792 90.067) (end 170.387 84.662) (width 0.2) (layer "F.Cu") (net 4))
 (segment (start 139.376 87.326) (end 137.174 87.326) (width 0.2) (layer "F.Cu") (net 4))
 (segment (start 166.37 78.105) (end 168.7925 78.105) (width 0.2) (layer "F.Cu") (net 4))
 (segment (start 179.759686 105.8585) (end 175.792 101.890814) (width 0.2) (layer "F.Cu") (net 4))
 (segment (start 183.826 85.951) (end 183.826 102.952814) (width 0.2) (layer "F.Cu") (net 4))
 (segment (start 167.64 77.7875) (end 167.9575 78.105) (width 0.2) (layer "B.Cu") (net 4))
 (segment (start 138.275 86.6) (end 139.299 85.576) (width 0.2) (layer "F.Cu") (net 1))
 (segment (start 179.225 84.85) (end 170.5795 76.2045) (width 0.2) (layer "F.Cu") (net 1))
 (segment (start 139.299 85.576) (end 139.376 85.576) (width 0.2) (layer "F.Cu") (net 1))
 (segment (start 138.275 86.6) (end 138.1125 86.7625) (width 0.2) (layer "F.Cu") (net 1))
 (segment (start 170.5795 76.2045) (end 148.6705 76.2045) (width 0.2) (layer "F.Cu") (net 1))
 (segment (start 139.376 85.576) (end 139.376 85.499) (width 0.2) (layer "F.Cu") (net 1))
 (segment (start 148.6705 76.2045) (end 138.275 86.6) (width 0.2) (layer "F.Cu") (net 1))
 (segment (start 173.27 80.645) (end 167.9575 80.645) (width 0.2) (layer "F.Cu") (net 2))
 (segment (start 179.225 86.6) (end 179.225 103.3425) (width 0.2) (layer "F.Cu") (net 2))
 (segment (start 179.225 86.6) (end 173.27 80.645) (width 0.2) (layer "F.Cu") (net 2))
 (segment (start 141.9225 104.775) (end 141.2875 104.775) (width 0.2) (layer "F.Cu") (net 2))
 (segment (start 179.225 103.3425) (end 180.34 104.4575) (width 0.2) (layer "F.Cu") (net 2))
 (segment (start 134.775 96.9925) (end 142.24 104.4575) (width 0.2) (layer "F.Cu") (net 2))
 (segment (start 134.775 86.6) (end 134.775 96.9925) (width 0.2) (layer "F.Cu") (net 2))
 (segment (start 161.29 104.4575) (end 161.29 123.5075) (width 0.2) (layer "B.Cu") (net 2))
 (segment (start 142.24 104.4575) (end 180.34 104.4575) (width 0.2) (layer "B.Cu") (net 2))
 (segment (start 142.24 104.4575) (end 142.24 123.5075) (width 0.2) (layer "B.Cu") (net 2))
 (segment (start 180.34 104.4575) (end 180.34 123.5075) (width 0.2) (layer "B.Cu") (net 2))
 (segment (start 141.681314 106.9975) (end 147.358157 101.320657) (width 0.2) (layer "F.Cu") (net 13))
 (segment (start 135.89 106.9975) (end 141.681314 106.9975) (width 0.2) (layer "F.Cu") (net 13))
 (segment (start 151.3575 90.28) (end 151.8825 90.805) (width 0.2) (layer "F.Cu") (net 13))
 (segment (start 147.358157 93.216843) (end 149.77 90.805) (width 0.2) (layer "F.Cu") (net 13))
 (segment (start 147.358157 101.320657) (end 147.358157 93.216843) (width 0.2) (layer "F.Cu") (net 13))
 (segment (start 149.77 90.805) (end 151.8825 90.805) (width 0.2) (layer "F.Cu") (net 13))
 (segment (start 151.13 110.8075) (end 151.13 92.82) (width 0.2) (layer "F.Cu") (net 14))
 (segment (start 151.13 92.5704) (end 151.13 92.82) (width 0.2) (layer "F.Cu") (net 14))
 (segment (start 135.89 126.0475) (end 151.13 110.8075) (width 0.2) (layer "F.Cu") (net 14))
 (segment (start 154.94 105.085) (end 154.94 106.9975) (width 0.2) (layer "F.Cu") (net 15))
 (segment (start 167.205 92.82) (end 167.4325 92.82) (width 0.2) (layer "F.Cu") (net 15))
 (segment (start 167.205 92.82) (end 154.94 105.085) (width 0.2) (layer "F.Cu") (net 15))
 (segment (start 167.4325 92.82) (end 167.9575 93.345) (width 0.2) (layer "F.Cu") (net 15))
 (segment (start 167.205 90.28) (end 168.722 91.797) (width 0.2) (layer "F.Cu") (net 7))
 (segment (start 171.45 109.5375) (end 171.45 93.4625) (width 0.2) (layer "F.Cu") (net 7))
 (segment (start 154.94 126.0475) (end 171.45 109.5375) (width 0.2) (layer "F.Cu") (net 7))
 (segment (start 171.45 93.4625) (end 168.7925 90.805) (width 0.2) (layer "F.Cu") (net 7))
 (segment (start 173.99 94.525) (end 173.99 106.9975) (width 0.2) (layer "F.Cu") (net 6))
 (segment (start 173.99 94.525) (end 173.99 93.4625) (width 0.2) (layer "F.Cu") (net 6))
 (segment (start 173.99 93.4625) (end 168.7925 88.265) (width 0.2) (layer "F.Cu") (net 6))
 (segment (start 168.7925 88.265) (end 167.9575 88.265) (width 0.2) (layer "F.Cu") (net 6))
 (segment (start 173.99 126.0475) (end 175.391 124.6465) (width 0.2) (layer "F.Cu") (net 16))
 (segment (start 175.391 92.3235) (end 168.7925 85.725) (width 0.2) (layer "F.Cu") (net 16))
 (segment (start 175.391 124.6465) (end 175.391 92.3235) (width 0.2) (layer "F.Cu") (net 16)))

